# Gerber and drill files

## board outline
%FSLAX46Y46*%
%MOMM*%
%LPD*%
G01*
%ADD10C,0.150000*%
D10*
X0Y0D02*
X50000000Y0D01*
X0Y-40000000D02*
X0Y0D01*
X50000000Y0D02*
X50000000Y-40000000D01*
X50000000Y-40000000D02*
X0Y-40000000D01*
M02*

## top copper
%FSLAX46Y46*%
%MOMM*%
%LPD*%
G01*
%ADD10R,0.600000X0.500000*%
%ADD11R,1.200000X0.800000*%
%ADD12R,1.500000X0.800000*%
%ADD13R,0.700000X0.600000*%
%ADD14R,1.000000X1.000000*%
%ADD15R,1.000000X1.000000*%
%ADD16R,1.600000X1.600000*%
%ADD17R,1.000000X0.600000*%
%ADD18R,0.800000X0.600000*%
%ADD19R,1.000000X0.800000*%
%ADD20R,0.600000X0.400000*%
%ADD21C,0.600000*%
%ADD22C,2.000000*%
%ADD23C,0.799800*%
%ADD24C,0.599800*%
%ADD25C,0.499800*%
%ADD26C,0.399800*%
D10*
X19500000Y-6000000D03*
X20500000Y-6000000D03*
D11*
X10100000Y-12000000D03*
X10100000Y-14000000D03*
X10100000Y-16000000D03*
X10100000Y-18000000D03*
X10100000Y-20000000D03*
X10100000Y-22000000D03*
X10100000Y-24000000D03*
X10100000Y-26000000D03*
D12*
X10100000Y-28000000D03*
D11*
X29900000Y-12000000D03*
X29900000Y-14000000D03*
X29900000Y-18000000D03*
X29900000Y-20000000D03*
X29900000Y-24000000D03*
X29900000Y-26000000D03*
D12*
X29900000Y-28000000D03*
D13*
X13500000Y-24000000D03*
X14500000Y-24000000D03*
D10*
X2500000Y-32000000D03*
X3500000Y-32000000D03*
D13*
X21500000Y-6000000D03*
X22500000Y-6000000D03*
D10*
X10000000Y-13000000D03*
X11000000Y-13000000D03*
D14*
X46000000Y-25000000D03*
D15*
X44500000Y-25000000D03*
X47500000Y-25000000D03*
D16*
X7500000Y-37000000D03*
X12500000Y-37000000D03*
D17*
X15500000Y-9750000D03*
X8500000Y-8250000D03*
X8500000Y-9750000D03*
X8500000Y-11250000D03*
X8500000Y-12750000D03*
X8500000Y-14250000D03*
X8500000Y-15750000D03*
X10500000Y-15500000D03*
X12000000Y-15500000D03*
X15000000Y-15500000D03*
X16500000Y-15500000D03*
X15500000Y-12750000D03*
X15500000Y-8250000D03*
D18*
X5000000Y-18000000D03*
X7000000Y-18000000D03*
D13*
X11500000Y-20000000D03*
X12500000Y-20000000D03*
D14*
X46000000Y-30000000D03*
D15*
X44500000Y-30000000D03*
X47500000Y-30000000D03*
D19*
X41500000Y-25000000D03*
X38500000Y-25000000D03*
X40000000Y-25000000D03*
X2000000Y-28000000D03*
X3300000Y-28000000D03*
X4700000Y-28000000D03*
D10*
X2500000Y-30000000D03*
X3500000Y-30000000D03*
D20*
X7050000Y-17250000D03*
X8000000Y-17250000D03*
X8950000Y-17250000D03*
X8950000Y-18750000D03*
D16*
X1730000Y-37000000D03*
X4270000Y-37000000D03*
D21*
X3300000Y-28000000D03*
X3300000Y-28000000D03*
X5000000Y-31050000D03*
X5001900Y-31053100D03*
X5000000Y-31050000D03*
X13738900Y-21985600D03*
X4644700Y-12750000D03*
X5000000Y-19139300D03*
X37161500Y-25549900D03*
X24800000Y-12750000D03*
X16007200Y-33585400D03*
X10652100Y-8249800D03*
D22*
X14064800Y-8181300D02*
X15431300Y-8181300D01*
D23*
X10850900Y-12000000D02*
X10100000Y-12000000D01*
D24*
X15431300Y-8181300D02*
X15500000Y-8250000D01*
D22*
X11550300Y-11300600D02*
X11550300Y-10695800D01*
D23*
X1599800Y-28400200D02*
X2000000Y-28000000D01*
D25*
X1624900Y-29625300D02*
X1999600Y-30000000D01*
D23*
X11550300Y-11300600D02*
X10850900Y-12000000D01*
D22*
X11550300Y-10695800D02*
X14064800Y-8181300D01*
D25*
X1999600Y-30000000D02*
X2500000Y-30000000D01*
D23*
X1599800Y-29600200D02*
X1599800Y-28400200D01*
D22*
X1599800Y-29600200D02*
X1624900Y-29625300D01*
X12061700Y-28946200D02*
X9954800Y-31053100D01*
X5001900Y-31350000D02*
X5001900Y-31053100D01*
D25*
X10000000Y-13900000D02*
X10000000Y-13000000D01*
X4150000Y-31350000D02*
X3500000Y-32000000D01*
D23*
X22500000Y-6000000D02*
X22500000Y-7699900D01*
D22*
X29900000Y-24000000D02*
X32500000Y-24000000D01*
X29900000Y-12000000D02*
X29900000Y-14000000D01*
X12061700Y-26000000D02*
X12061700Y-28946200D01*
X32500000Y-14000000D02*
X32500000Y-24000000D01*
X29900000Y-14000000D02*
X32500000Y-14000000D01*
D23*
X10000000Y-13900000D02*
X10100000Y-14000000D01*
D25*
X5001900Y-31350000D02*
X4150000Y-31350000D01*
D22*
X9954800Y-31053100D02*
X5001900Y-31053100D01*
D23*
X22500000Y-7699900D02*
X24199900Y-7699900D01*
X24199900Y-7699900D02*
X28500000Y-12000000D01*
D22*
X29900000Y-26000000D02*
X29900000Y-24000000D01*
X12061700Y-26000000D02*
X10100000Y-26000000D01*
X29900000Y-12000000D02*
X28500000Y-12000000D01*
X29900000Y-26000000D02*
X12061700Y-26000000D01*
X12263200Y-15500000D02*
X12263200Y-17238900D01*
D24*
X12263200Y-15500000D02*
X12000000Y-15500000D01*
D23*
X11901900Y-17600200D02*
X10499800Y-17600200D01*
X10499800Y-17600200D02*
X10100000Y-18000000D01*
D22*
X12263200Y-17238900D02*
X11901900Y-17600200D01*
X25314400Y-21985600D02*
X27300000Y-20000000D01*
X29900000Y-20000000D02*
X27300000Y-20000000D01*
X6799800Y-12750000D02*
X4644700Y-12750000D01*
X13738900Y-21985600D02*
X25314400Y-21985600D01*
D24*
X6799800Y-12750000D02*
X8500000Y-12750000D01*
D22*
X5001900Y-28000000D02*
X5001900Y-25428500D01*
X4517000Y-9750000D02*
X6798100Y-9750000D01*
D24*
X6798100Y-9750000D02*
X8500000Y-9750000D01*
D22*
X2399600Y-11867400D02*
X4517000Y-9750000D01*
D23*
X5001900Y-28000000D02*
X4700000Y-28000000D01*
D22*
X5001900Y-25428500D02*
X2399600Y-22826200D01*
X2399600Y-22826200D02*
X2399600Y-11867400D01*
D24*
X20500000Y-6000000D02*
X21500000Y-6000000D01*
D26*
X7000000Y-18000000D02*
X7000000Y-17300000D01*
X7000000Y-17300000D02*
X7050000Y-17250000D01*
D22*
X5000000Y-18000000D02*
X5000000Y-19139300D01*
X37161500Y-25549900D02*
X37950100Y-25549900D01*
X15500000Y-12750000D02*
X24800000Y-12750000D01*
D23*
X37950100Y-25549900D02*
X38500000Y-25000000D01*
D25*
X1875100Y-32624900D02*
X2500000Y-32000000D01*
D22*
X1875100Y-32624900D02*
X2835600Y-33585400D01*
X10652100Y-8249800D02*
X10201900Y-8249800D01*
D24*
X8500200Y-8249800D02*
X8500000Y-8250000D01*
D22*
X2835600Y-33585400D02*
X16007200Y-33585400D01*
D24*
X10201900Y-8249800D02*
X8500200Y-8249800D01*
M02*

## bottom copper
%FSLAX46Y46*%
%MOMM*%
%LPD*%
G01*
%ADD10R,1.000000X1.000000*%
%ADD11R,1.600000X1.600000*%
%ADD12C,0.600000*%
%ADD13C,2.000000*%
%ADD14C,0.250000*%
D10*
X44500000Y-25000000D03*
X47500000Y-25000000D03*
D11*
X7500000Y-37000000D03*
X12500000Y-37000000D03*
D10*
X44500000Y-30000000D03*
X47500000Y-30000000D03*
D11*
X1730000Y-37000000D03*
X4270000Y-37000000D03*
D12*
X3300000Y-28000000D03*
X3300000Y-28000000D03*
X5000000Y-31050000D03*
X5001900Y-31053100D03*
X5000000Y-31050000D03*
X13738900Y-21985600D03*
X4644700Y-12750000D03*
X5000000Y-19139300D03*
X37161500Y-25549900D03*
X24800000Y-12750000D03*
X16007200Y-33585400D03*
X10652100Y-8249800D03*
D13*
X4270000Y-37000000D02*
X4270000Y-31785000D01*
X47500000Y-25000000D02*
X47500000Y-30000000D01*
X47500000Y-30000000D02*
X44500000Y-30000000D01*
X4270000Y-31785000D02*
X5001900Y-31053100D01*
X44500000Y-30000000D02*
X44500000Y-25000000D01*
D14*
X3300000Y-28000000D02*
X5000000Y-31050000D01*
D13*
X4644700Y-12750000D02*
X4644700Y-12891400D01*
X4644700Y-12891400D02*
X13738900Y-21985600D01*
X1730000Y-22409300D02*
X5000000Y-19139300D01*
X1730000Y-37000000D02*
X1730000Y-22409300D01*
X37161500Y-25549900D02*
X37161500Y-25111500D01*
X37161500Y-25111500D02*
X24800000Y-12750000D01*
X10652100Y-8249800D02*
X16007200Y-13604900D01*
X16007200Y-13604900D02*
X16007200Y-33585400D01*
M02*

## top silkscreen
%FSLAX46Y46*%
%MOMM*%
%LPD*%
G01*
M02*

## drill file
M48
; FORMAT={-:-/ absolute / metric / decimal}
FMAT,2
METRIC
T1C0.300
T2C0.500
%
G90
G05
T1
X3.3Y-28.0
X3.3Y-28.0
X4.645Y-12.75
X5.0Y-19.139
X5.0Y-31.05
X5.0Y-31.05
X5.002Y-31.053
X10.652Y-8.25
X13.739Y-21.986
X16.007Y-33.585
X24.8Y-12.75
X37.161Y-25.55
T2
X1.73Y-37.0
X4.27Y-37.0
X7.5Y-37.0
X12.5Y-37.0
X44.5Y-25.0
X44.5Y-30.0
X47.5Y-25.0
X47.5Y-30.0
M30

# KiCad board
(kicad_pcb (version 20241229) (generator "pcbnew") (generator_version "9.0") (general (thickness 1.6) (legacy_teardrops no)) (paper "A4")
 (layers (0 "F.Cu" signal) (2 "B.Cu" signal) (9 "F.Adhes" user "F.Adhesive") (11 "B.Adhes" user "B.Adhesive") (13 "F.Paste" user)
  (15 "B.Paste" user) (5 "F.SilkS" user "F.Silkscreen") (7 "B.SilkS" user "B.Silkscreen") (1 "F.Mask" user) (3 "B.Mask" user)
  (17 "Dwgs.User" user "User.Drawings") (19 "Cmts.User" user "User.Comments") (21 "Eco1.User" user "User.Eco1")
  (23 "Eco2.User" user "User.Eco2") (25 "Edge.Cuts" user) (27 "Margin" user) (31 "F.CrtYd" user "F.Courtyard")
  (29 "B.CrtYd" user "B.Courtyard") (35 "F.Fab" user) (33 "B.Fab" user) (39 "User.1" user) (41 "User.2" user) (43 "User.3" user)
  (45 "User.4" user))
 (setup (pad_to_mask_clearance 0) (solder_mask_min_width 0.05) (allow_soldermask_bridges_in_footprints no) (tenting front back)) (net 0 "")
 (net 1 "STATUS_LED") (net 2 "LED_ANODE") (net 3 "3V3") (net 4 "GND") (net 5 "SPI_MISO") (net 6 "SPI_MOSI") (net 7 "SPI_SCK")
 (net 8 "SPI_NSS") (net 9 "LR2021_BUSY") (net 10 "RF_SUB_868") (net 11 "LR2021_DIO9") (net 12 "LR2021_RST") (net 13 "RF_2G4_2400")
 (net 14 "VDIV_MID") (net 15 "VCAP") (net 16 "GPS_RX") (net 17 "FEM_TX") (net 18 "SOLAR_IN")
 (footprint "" (layer "F.Cu") (at 20 6)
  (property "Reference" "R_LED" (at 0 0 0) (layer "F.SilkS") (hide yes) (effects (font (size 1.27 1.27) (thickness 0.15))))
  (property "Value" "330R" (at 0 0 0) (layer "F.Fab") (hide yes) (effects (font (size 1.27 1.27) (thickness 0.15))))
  (pad "1" smd rect (at -0.5 0) (size 0.6 0.5) (layers "F.Cu" "F.Mask") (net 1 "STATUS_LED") (thermal_bridge_angle 45))
  (pad "2" smd rect (at 0.5 0) (size 0.6 0.5) (layers "F.Cu" "F.Mask") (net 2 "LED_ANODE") (thermal_bridge_angle 45)))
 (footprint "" (layer "F.Cu") (at 20 20)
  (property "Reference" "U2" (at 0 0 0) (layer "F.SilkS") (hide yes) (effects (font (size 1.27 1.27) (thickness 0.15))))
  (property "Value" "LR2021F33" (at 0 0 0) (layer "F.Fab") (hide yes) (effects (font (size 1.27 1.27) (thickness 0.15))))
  (pad "1" smd rect (at -9.9 -8) (size 1.2 0.8) (layers "F.Cu" "F.Mask") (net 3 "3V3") (thermal_bridge_angle 45))
  (pad "2" smd rect (at -9.9 -6) (size 1.2 0.8) (layers "F.Cu" "F.Mask") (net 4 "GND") (thermal_bridge_angle 45))
  (pad "3" smd rect (at -9.9 -4) (size 1.2 0.8) (layers "F.Cu" "F.Mask") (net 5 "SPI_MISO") (thermal_bridge_angle 45))
  (pad "4" smd rect (at -9.9 -2) (size 1.2 0.8) (layers "F.Cu" "F.Mask") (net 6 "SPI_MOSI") (thermal_bridge_angle 45))
  (pad "5" smd rect (at -9.9 0) (size 1.2 0.8) (layers "F.Cu" "F.Mask") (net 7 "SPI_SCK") (thermal_bridge_angle 45))
  (pad "6" smd rect (at -9.9 2) (size 1.2 0.8) (layers "F.Cu" "F.Mask") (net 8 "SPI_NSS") (thermal_bridge_angle 45))
  (pad "7" smd rect (at -9.9 4) (size 1.2 0.8) (layers "F.Cu" "F.Mask") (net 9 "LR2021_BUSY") (thermal_bridge_angle 45))
  (pad "8" smd rect (at -9.9 6) (size 1.2 0.8) (layers "F.Cu" "F.Mask") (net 4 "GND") (thermal_bridge_angle 45))
  (pad "9" smd rect (at -9.9 8) (size 1.5 0.8) (layers "F.Cu" "F.Mask") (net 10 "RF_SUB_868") (thermal_bridge_angle 45))
  (pad "10" smd rect (at 9.9 -8) (size 1.2 0.8) (layers "F.Cu" "F.Mask") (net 4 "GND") (thermal_bridge_angle 45))
  (pad "11" smd rect (at 9.9 -6) (size 1.2 0.8) (layers "F.Cu" "F.Mask") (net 4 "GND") (thermal_bridge_angle 45))
  (pad "13" smd rect (at 9.9 -2) (size 1.2 0.8) (layers "F.Cu" "F.Mask") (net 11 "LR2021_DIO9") (thermal_bridge_angle 45))
  (pad "14" smd rect (at 9.9 0) (size 1.2 0.8) (layers "F.Cu" "F.Mask") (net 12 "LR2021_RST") (thermal_bridge_angle 45))
  (pad "16" smd rect (at 9.9 4) (size 1.2 0.8) (layers "F.Cu" "F.Mask") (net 4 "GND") (thermal_bridge_angle 45))
  (pad "17" smd rect (at 9.9 6) (size 1.2 0.8) (layers "F.Cu" "F.Mask") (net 4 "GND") (thermal_bridge_angle 45))
  (pad "18" smd rect (at 9.9 8) (size 1.5 0.8) (layers "F.Cu" "F.Mask") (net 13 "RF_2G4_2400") (thermal_bridge_angle 45)))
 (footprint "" (layer "F.Cu") (at 14 24)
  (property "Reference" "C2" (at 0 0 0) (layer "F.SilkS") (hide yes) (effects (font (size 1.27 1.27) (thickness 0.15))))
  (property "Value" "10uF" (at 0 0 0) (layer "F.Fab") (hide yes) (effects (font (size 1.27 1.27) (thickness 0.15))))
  (pad "1" smd rect (at -0.5 0) (size 0.7 0.6) (layers "F.Cu" "F.Mask") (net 3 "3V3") (thermal_bridge_angle 45))
  (pad "2" smd rect (at 0.5 0) (size 0.7 0.6) (layers "F.Cu" "F.Mask") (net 4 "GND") (thermal_bridge_angle 45)))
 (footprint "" (layer "F.Cu") (at 3 32)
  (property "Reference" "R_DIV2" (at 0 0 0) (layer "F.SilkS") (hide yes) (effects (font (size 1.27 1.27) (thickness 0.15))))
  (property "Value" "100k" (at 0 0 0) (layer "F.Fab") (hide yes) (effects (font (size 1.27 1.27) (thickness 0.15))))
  (pad "1" smd rect (at -0.5 0) (size 0.6 0.5) (layers "F.Cu" "F.Mask") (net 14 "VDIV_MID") (thermal_bridge_angle 45))
  (pad "2" smd rect (at 0.5 0) (size 0.6 0.5) (layers "F.Cu" "F.Mask") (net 4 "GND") (thermal_bridge_angle 45)))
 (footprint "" (layer "F.Cu") (at 22 6)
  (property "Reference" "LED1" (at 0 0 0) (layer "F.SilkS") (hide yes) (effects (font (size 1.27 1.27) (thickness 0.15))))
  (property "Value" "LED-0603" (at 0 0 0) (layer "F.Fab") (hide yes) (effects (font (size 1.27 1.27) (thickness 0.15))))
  (pad "A" smd rect (at -0.5 0) (size 0.7 0.6) (layers "F.Cu" "F.Mask") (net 2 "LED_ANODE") (thermal_bridge_angle 45))
  (pad "K" smd rect (at 0.5 0) (size 0.7 0.6) (layers "F.Cu" "F.Mask") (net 4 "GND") (thermal_bridge_angle 45)))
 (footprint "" (layer "F.Cu") (at 10.5 13)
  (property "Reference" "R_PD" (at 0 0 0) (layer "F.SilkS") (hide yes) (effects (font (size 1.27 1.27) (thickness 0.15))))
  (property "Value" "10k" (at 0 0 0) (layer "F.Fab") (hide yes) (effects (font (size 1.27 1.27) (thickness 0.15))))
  (pad "1" smd rect (at -0.5 0) (size 0.6 0.5) (layers "F.Cu" "F.Mask") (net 4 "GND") (thermal_bridge_angle 45))
  (pad "2" smd rect (at 0.5 0) (size 0.6 0.5) (layers "F.Cu" "F.Mask") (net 5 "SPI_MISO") (thermal_bridge_angle 45)))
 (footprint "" (layer "F.Cu") (at 46 25)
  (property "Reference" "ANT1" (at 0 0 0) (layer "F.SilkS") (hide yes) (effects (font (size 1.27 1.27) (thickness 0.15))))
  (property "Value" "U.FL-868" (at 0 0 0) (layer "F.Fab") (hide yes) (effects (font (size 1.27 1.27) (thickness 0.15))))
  (pad "1" smd rect (at 0 0) (size 1 1) (layers "F.Cu" "F.Mask") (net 10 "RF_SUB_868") (thermal_bridge_angle 45))
  (pad "2" thru_hole rect (at -1.5 0) (size 1 1) (drill 0.5) (layers "*.Cu" "*.Mask") (remove_unused_layers no) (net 4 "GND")
   (thermal_bridge_angle 45))
  (pad "3" thru_hole rect (at 1.5 0) (size 1 1) (drill 0.5) (layers "*.Cu" "*.Mask") (remove_unused_layers no) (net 4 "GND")
   (thermal_bridge_angle 45)))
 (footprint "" (layer "F.Cu") (at 10 37)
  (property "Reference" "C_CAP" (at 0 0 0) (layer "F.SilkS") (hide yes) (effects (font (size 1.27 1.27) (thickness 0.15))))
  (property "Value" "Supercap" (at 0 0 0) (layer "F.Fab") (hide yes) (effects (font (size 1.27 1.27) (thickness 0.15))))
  (pad "1" thru_hole rect (at -2.5 0) (size 1.6 1.6) (drill 0.5) (layers "*.Cu" "*.Mask") (remove_unused_layers no) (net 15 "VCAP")
   (thermal_bridge_angle 45))
  (pad "2" thru_hole rect (at 2.5 0) (size 1.6 1.6) (drill 0.5) (layers "*.Cu" "*.Mask") (remove_unused_layers no) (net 4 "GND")
   (thermal_bridge_angle 45)))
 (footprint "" (layer "F.Cu") (at 12 12)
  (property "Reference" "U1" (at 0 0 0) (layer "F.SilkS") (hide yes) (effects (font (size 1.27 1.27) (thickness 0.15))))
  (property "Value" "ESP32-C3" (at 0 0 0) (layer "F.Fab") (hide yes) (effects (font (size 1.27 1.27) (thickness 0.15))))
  (pad "GND" smd rect (at 3.5 -2.25) (size 1 0.6) (layers "F.Cu" "F.Mask") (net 4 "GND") (thermal_bridge_angle 45))
  (pad "GPIO0" smd rect (at -3.5 -3.75) (size 1 0.6) (layers "F.Cu" "F.Mask") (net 14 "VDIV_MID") (thermal_bridge_angle 45))
  (pad "GPIO1" smd rect (at -3.5 -2.25) (size 1 0.6) (layers "F.Cu" "F.Mask") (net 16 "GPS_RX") (thermal_bridge_angle 45))
  (pad "GPIO2" smd rect (at -3.5 -0.75) (size 1 0.6) (layers "F.Cu" "F.Mask") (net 5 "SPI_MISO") (thermal_bridge_angle 45))
  (pad "GPIO3" smd rect (at -3.5 0.75) (size 1 0.6) (layers "F.Cu" "F.Mask") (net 12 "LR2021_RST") (thermal_bridge_angle 45))
  (pad "GPIO4" smd rect (at -3.5 2.25) (size 1 0.6) (layers "F.Cu" "F.Mask") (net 9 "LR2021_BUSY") (thermal_bridge_angle 45))
  (pad "GPIO5" smd rect (at -3.5 3.75) (size 1 0.6) (layers "F.Cu" "F.Mask") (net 11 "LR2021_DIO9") (thermal_bridge_angle 45))
  (pad "GPIO6" smd rect (at -1.5 3.5) (size 1 0.6) (layers "F.Cu" "F.Mask") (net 7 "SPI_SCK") (thermal_bridge_angle 45))
  (pad "GPIO7" smd rect (at 0 3.5) (size 1 0.6) (layers "F.Cu" "F.Mask") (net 6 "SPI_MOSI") (thermal_bridge_angle 45))
  (pad "GPIO9" smd rect (at 3 3.5) (size 1 0.6) (layers "F.Cu" "F.Mask") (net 1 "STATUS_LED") (thermal_bridge_angle 45))
  (pad "GPIO10" smd rect (at 4.5 3.5) (size 1 0.6) (layers "F.Cu" "F.Mask") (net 8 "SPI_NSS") (thermal_bridge_angle 45))
  (pad "GPIO19" smd rect (at 3.5 0.75) (size 1 0.6) (layers "F.Cu" "F.Mask") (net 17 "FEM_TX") (thermal_bridge_angle 45))
  (pad "VCC" smd rect (at 3.5 -3.75) (size 1 0.6) (layers "F.Cu" "F.Mask") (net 3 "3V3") (thermal_bridge_angle 45)))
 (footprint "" (layer "F.Cu") (at 6 18)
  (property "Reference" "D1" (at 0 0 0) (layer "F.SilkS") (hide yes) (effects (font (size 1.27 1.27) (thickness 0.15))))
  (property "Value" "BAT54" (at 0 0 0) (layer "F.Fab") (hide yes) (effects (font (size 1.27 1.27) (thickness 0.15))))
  (pad "A" smd rect (at -1 0) (size 0.8 0.6) (layers "F.Cu" "F.Mask") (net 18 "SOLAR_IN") (thermal_bridge_angle 45))
  (pad "K" smd rect (at 1 0) (size 0.8 0.6) (layers "F.Cu" "F.Mask") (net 15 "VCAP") (thermal_bridge_angle 45)))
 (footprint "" (layer "F.Cu") (at 12 20)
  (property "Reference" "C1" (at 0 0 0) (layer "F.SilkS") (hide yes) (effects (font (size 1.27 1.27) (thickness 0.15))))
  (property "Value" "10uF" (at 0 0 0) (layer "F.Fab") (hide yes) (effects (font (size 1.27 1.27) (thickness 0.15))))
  (pad "1" smd rect (at -0.5 0) (size 0.7 0.6) (layers "F.Cu" "F.Mask") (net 15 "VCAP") (thermal_bridge_angle 45))
  (pad "2" smd rect (at 0.5 0) (size 0.7 0.6) (layers "F.Cu" "F.Mask") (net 4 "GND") (thermal_bridge_angle 45)))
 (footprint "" (layer "F.Cu") (at 46 30)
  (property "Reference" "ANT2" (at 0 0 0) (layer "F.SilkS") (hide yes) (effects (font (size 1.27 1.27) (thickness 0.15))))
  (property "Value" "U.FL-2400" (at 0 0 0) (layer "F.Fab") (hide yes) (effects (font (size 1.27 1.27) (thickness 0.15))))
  (pad "1" smd rect (at 0 0) (size 1 1) (layers "F.Cu" "F.Mask") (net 13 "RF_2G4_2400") (thermal_bridge_angle 45))
  (pad "2" thru_hole rect (at -1.5 0) (size 1 1) (drill 0.5) (layers "*.Cu" "*.Mask") (remove_unused_layers no) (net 4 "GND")
   (thermal_bridge_angle 45))
  (pad "3" thru_hole rect (at 1.5 0) (size 1 1) (drill 0.5) (layers "*.Cu" "*.Mask") (remove_unused_layers no) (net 4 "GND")
   (thermal_bridge_angle 45)))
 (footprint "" (layer "F.Cu") (at 40 25)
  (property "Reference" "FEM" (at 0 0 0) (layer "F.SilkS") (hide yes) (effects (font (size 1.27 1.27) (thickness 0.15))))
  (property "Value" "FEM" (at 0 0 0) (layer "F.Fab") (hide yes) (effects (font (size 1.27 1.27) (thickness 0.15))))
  (pad "GND" smd rect (at 1.5 0) (size 1 0.8) (layers "F.Cu" "F.Mask") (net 4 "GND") (thermal_bridge_angle 45))
  (pad "TX" smd rect (at -1.5 0) (size 1 0.8) (layers "F.Cu" "F.Mask") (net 17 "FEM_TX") (thermal_bridge_angle 45))
  (pad "VCC" smd rect (at 0 0) (size 1 0.8) (layers "F.Cu" "F.Mask") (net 3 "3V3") (thermal_bridge_angle 45)))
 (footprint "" (layer "F.Cu") (at 4 28)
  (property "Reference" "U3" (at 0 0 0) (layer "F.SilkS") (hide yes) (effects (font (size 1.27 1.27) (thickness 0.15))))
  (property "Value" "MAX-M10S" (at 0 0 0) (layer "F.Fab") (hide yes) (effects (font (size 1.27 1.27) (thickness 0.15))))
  (pad "1" smd rect (at -2 0) (size 1 0.8) (layers "F.Cu" "F.Mask") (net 3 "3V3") (thermal_bridge_angle 45))
  (pad "2" smd rect (at -0.7 0) (size 1 0.8) (layers "F.Cu" "F.Mask") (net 4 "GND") (thermal_bridge_angle 45))
  (pad "3" smd rect (at 0.7 0) (size 1 0.8) (layers "F.Cu" "F.Mask") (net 16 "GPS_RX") (thermal_bridge_angle 45)))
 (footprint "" (layer "F.Cu") (at 3 30)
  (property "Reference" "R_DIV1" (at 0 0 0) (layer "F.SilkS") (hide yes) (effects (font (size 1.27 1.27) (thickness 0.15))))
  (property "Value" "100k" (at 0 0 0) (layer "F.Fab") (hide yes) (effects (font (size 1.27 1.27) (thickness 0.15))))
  (pad "1" smd rect (at -0.5 0) (size 0.6 0.5) (layers "F.Cu" "F.Mask") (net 3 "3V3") (thermal_bridge_angle 45))
  (pad "2" smd rect (at 0.5 0) (size 0.6 0.5) (layers "F.Cu" "F.Mask") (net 14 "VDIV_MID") (thermal_bridge_angle 45)))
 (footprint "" (layer "F.Cu") (at 8 18)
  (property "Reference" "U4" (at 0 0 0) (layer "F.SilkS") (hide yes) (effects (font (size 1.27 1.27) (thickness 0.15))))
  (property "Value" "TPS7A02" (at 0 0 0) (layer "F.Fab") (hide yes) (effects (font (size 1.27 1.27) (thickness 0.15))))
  (pad "1" smd rect (at -0.95 -0.75) (size 0.6 0.4) (layers "F.Cu" "F.Mask") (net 15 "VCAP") (thermal_bridge_angle 45))
  (pad "2" smd rect (at 0 -0.75) (size 0.6 0.4) (layers "F.Cu" "F.Mask") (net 4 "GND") (thermal_bridge_angle 45))
  (pad "3" smd rect (at 0.95 -0.75) (size 0.6 0.4) (layers "F.Cu" "F.Mask") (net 15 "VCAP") (thermal_bridge_angle 45))
  (pad "4" smd rect (at 0.95 0.75) (size 0.6 0.4) (layers "F.Cu" "F.Mask") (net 3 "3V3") (thermal_bridge_angle 45)))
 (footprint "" (layer "F.Cu") (at 3 37)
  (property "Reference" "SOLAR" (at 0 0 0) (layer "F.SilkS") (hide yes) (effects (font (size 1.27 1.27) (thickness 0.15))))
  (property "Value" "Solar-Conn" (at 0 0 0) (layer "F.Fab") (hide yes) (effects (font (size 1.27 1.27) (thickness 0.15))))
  (pad "1" thru_hole rect (at -1.27 0) (size 1.6 1.6) (drill 0.5) (layers "*.Cu" "*.Mask") (remove_unused_layers no) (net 18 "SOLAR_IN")
   (thermal_bridge_angle 45))
  (pad "2" thru_hole rect (at 1.27 0) (size 1.6 1.6) (drill 0.5) (layers "*.Cu" "*.Mask") (remove_unused_layers no) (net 4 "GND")
   (thermal_bridge_angle 45)))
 (gr_line (start 0 0) (end 50 0) (stroke (width 0.15) (type default)) (layer "Edge.Cuts"))
 (gr_line (start 0 40) (end 0 0) (stroke (width 0.15) (type default)) (layer "Edge.Cuts"))
 (gr_line (start 50 0) (end 50 40) (stroke (width 0.15) (type default)) (layer "Edge.Cuts"))
 (gr_line (start 50 40) (end 0 40) (stroke (width 0.15) (type default)) (layer "Edge.Cuts"))
 (segment (start 14.0648 8.1813) (end 15.4313 8.1813) (width 2) (layer "F.Cu") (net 3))
 (segment (start 10.8509 12) (end 10.1 12) (width 0.7998) (layer "F.Cu") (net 3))
 (segment (start 15.4313 8.1813) (end 15.5 8.25) (width 0.5998) (layer "F.Cu") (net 3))
 (segment (start 11.5503 11.3006) (end 11.5503 10.6958) (width 2) (layer "F.Cu") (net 3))
 (segment (start 1.5998 28.4002) (end 2 28) (width 0.7998) (layer "F.Cu") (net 3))
 (segment (start 1.6249 29.6253) (end 1.9996 30) (width 0.4998) (layer "F.Cu") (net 3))
 (segment (start 11.5503 11.3006) (end 10.8509 12) (width 0.7998) (layer "F.Cu") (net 3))
 (segment (start 11.5503 10.6958) (end 14.0648 8.1813) (width 2) (layer "F.Cu") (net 3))
 (segment (start 1.9996 30) (end 2.5 30) (width 0.4998) (layer "F.Cu") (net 3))
 (segment (start 1.5998 29.6002) (end 1.5998 28.4002) (width 0.7998) (layer "F.Cu") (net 3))
 (segment (start 1.5998 29.6002) (end 1.6249 29.6253) (width 2) (layer "F.Cu") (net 3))
 (segment (start 12.0617 28.9462) (end 9.9548 31.0531) (width 2) (layer "F.Cu") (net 4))
 (segment (start 5.0019 31.35) (end 5.0019 31.0531) (width 2) (layer "F.Cu") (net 4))
 (segment (start 10 13.9) (end 10 13) (width 0.4998) (layer "F.Cu") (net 4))
 (segment (start 4.15 31.35) (end 3.5 32) (width 0.4998) (layer "F.Cu") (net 4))
 (segment (start 22.5 6) (end 22.5 7.6999) (width 0.7998) (layer "F.Cu") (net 4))
 (segment (start 29.9 24) (end 32.5 24) (width 2) (layer "F.Cu") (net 4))
 (segment (start 29.9 12) (end 29.9 14) (width 2) (layer "F.Cu") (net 4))
 (segment (start 12.0617 26) (end 12.0617 28.9462) (width 2) (layer "F.Cu") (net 4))
 (segment (start 32.5 14) (end 32.5 24) (width 2) (layer "F.Cu") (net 4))
 (segment (start 29.9 14) (end 32.5 14) (width 2) (layer "F.Cu") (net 4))
 (segment (start 10 13.9) (end 10.1 14) (width 0.7998) (layer "F.Cu") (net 4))
 (segment (start 5.0019 31.35) (end 4.15 31.35) (width 0.4998) (layer "F.Cu") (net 4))
 (segment (start 9.9548 31.0531) (end 5.0019 31.0531) (width 2) (layer "F.Cu") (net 4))
 (segment (start 22.5 7.6999) (end 24.1999 7.6999) (width 0.7998) (layer "F.Cu") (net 4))
 (segment (start 24.1999 7.6999) (end 28.5 12) (width 0.7998) (layer "F.Cu") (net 4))
 (segment (start 29.9 26) (end 29.9 24) (width 2) (layer "F.Cu") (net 4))
 (segment (start 12.0617 26) (end 10.1 26) (width 2) (layer "F.Cu") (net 4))
 (segment (start 29.9 12) (end 28.5 12) (width 2) (layer "F.Cu") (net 4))
 (segment (start 29.9 26) (end 12.0617 26) (width 2) (layer "F.Cu") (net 4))
 (via (at 3.3 28) (size 0.6) (drill 0.3) (layers "F.Cu" "B.Cu") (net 4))
 (via (at 3.3 28) (size 0.6) (drill 0.3) (layers "F.Cu" "B.Cu") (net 4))
 (via (at 5 31.05) (size 0.6) (drill 0.3) (layers "F.Cu" "B.Cu") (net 4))
 (via (at 5.0019 31.0531) (size 0.6) (drill 0.3) (layers "F.Cu" "B.Cu") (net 4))
 (via (at 5 31.05) (size 0.6) (drill 0.3) (layers "F.Cu" "B.Cu") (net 4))
 (segment (start 4.27 37) (end 4.27 31.785) (width 2) (layer "B.Cu") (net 4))
 (segment (start 47.5 25) (end 47.5 30) (width 2) (layer "B.Cu") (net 4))
 (segment (start 47.5 30) (end 44.5 30) (width 2) (layer "B.Cu") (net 4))
 (segment (start 4.27 31.785) (end 5.0019 31.0531) (width 2) (layer "B.Cu") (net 4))
 (segment (start 44.5 30) (end 44.5 25) (width 2) (layer "B.Cu") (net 4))
 (segment (start 3.3 28) (end 5 31.05) (width 0.25) (layer "B.Cu") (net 4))
 (segment (start 12.2632 15.5) (end 12.2632 17.2389) (width 2) (layer "F.Cu") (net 6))
 (segment (start 12.2632 15.5) (end 12 15.5) (width 0.5998) (layer "F.Cu") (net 6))
 (segment (start 11.9019 17.6002) (end 10.4998 17.6002) (width 0.7998) (layer "F.Cu") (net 6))
 (segment (start 10.4998 17.6002) (end 10.1 18) (width 0.7998) (layer "F.Cu") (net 6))
 (segment (start 12.2632 17.2389) (end 11.9019 17.6002) (width 2) (layer "F.Cu") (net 6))
 (segment (start 25.3144 21.9856) (end 27.3 20) (width 2) (layer "F.Cu") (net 12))
 (segment (start 29.9 20) (end 27.3 20) (width 2) (layer "F.Cu") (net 12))
 (segment (start 6.7998 12.75) (end 4.6447 12.75) (width 2) (layer "F.Cu") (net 12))
 (segment (start 13.7389 21.9856) (end 25.3144 21.9856) (width 2) (layer "F.Cu") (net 12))
 (segment (start 6.7998 12.75) (end 8.5 12.75) (width 0.5998) (layer "F.Cu") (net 12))
 (via (at 13.7389 21.9856) (size 0.6) (drill 0.3) (layers "F.Cu" "B.Cu") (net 12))
 (via (at 4.6447 12.75) (size 0.6) (drill 0.3) (layers "F.Cu" "B.Cu") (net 12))
 (segment (start 4.6447 12.75) (end 4.6447 12.8914) (width 2) (layer "B.Cu") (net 12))
 (segment (start 4.6447 12.8914) (end 13.7389 21.9856) (width 2) (layer "B.Cu") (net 12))
 (segment (start 5.0019 28) (end 5.0019 25.4285) (width 2) (layer "F.Cu") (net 16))
 (segment (start 4.517 9.75) (end 6.7981 9.75) (width 2) (layer "F.Cu") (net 16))
 (segment (start 6.7981 9.75) (end 8.5 9.75) (width 0.5998) (layer "F.Cu") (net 16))
 (segment (start 2.3996 11.8674) (end 4.517 9.75) (width 2) (layer "F.Cu") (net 16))
 (segment (start 5.0019 28) (end 4.7 28) (width 0.7998) (layer "F.Cu") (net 16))
 (segment (start 5.0019 25.4285) (end 2.3996 22.8262) (width 2) (layer "F.Cu") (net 16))
 (segment (start 2.3996 22.8262) (end 2.3996 11.8674) (width 2) (layer "F.Cu") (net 16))
 (segment (start 20.5 6) (end 21.5 6) (width 0.5998) (layer "F.Cu") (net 2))
 (segment (start 7 18) (end 7 17.3) (width 0.3998) (layer "F.Cu") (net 15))
 (segment (start 7 17.3) (end 7.05 17.25) (width 0.3998) (layer "F.Cu") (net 15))
 (segment (start 5 18) (end 5 19.1393) (width 2) (layer "F.Cu") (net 18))
 (via (at 5 19.1393) (size 0.6) (drill 0.3) (layers "F.Cu" "B.Cu") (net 18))
 (segment (start 1.73 22.4093) (end 5 19.1393) (width 2) (layer "B.Cu") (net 18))
 (segment (start 1.73 37) (end 1.73 22.4093) (width 2) (layer "B.Cu") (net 18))
 (segment (start 37.1615 25.5499) (end 37.9501 25.5499) (width 2) (layer "F.Cu") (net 17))
 (segment (start 15.5 12.75) (end 24.8 12.75) (width 2) (layer "F.Cu") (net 17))
 (segment (start 37.9501 25.5499) (end 38.5 25) (width 0.7998) (layer "F.Cu") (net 17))
 (via (at 37.1615 25.5499) (size 0.6) (drill 0.3) (layers "F.Cu" "B.Cu") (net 17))
 (via (at 24.8 12.75) (size 0.6) (drill 0.3) (layers "F.Cu" "B.Cu") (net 17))
 (segment (start 37.1615 25.5499) (end 37.1615 25.1115) (width 2) (layer "B.Cu") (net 17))
 (segment (start 37.1615 25.1115) (end 24.8 12.75) (width 2) (layer "B.Cu") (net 17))
 (segment (start 1.8751 32.6249) (end 2.5 32) (width 0.4998) (layer "F.Cu") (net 14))
 (segment (start 1.8751 32.6249) (end 2.8356 33.5854) (width 2) (layer "F.Cu") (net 14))
 (segment (start 10.6521 8.2498) (end 10.2019 8.2498) (width 2) (layer "F.Cu") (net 14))
 (segment (start 8.5002 8.2498) (end 8.5 8.25) (width 0.5998) (layer "F.Cu") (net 14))
 (segment (start 2.8356 33.5854) (end 16.0072 33.5854) (width 2) (layer "F.Cu") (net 14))
 (segment (start 10.2019 8.2498) (end 8.5002 8.2498) (width 0.5998) (layer "F.Cu") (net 14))
 (via (at 16.0072 33.5854) (size 0.6) (drill 0.3) (layers "F.Cu" "B.Cu") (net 14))
 (via (at 10.6521 8.2498) (size 0.6) (drill 0.3) (layers "F.Cu" "B.Cu") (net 14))
 (segment (start 10.6521 8.2498) (end 16.0072 13.6049) (width 2) (layer "B.Cu") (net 14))
 (segment (start 16.0072 13.6049) (end 16.0072 33.5854) (width 2) (layer "B.Cu") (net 14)))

